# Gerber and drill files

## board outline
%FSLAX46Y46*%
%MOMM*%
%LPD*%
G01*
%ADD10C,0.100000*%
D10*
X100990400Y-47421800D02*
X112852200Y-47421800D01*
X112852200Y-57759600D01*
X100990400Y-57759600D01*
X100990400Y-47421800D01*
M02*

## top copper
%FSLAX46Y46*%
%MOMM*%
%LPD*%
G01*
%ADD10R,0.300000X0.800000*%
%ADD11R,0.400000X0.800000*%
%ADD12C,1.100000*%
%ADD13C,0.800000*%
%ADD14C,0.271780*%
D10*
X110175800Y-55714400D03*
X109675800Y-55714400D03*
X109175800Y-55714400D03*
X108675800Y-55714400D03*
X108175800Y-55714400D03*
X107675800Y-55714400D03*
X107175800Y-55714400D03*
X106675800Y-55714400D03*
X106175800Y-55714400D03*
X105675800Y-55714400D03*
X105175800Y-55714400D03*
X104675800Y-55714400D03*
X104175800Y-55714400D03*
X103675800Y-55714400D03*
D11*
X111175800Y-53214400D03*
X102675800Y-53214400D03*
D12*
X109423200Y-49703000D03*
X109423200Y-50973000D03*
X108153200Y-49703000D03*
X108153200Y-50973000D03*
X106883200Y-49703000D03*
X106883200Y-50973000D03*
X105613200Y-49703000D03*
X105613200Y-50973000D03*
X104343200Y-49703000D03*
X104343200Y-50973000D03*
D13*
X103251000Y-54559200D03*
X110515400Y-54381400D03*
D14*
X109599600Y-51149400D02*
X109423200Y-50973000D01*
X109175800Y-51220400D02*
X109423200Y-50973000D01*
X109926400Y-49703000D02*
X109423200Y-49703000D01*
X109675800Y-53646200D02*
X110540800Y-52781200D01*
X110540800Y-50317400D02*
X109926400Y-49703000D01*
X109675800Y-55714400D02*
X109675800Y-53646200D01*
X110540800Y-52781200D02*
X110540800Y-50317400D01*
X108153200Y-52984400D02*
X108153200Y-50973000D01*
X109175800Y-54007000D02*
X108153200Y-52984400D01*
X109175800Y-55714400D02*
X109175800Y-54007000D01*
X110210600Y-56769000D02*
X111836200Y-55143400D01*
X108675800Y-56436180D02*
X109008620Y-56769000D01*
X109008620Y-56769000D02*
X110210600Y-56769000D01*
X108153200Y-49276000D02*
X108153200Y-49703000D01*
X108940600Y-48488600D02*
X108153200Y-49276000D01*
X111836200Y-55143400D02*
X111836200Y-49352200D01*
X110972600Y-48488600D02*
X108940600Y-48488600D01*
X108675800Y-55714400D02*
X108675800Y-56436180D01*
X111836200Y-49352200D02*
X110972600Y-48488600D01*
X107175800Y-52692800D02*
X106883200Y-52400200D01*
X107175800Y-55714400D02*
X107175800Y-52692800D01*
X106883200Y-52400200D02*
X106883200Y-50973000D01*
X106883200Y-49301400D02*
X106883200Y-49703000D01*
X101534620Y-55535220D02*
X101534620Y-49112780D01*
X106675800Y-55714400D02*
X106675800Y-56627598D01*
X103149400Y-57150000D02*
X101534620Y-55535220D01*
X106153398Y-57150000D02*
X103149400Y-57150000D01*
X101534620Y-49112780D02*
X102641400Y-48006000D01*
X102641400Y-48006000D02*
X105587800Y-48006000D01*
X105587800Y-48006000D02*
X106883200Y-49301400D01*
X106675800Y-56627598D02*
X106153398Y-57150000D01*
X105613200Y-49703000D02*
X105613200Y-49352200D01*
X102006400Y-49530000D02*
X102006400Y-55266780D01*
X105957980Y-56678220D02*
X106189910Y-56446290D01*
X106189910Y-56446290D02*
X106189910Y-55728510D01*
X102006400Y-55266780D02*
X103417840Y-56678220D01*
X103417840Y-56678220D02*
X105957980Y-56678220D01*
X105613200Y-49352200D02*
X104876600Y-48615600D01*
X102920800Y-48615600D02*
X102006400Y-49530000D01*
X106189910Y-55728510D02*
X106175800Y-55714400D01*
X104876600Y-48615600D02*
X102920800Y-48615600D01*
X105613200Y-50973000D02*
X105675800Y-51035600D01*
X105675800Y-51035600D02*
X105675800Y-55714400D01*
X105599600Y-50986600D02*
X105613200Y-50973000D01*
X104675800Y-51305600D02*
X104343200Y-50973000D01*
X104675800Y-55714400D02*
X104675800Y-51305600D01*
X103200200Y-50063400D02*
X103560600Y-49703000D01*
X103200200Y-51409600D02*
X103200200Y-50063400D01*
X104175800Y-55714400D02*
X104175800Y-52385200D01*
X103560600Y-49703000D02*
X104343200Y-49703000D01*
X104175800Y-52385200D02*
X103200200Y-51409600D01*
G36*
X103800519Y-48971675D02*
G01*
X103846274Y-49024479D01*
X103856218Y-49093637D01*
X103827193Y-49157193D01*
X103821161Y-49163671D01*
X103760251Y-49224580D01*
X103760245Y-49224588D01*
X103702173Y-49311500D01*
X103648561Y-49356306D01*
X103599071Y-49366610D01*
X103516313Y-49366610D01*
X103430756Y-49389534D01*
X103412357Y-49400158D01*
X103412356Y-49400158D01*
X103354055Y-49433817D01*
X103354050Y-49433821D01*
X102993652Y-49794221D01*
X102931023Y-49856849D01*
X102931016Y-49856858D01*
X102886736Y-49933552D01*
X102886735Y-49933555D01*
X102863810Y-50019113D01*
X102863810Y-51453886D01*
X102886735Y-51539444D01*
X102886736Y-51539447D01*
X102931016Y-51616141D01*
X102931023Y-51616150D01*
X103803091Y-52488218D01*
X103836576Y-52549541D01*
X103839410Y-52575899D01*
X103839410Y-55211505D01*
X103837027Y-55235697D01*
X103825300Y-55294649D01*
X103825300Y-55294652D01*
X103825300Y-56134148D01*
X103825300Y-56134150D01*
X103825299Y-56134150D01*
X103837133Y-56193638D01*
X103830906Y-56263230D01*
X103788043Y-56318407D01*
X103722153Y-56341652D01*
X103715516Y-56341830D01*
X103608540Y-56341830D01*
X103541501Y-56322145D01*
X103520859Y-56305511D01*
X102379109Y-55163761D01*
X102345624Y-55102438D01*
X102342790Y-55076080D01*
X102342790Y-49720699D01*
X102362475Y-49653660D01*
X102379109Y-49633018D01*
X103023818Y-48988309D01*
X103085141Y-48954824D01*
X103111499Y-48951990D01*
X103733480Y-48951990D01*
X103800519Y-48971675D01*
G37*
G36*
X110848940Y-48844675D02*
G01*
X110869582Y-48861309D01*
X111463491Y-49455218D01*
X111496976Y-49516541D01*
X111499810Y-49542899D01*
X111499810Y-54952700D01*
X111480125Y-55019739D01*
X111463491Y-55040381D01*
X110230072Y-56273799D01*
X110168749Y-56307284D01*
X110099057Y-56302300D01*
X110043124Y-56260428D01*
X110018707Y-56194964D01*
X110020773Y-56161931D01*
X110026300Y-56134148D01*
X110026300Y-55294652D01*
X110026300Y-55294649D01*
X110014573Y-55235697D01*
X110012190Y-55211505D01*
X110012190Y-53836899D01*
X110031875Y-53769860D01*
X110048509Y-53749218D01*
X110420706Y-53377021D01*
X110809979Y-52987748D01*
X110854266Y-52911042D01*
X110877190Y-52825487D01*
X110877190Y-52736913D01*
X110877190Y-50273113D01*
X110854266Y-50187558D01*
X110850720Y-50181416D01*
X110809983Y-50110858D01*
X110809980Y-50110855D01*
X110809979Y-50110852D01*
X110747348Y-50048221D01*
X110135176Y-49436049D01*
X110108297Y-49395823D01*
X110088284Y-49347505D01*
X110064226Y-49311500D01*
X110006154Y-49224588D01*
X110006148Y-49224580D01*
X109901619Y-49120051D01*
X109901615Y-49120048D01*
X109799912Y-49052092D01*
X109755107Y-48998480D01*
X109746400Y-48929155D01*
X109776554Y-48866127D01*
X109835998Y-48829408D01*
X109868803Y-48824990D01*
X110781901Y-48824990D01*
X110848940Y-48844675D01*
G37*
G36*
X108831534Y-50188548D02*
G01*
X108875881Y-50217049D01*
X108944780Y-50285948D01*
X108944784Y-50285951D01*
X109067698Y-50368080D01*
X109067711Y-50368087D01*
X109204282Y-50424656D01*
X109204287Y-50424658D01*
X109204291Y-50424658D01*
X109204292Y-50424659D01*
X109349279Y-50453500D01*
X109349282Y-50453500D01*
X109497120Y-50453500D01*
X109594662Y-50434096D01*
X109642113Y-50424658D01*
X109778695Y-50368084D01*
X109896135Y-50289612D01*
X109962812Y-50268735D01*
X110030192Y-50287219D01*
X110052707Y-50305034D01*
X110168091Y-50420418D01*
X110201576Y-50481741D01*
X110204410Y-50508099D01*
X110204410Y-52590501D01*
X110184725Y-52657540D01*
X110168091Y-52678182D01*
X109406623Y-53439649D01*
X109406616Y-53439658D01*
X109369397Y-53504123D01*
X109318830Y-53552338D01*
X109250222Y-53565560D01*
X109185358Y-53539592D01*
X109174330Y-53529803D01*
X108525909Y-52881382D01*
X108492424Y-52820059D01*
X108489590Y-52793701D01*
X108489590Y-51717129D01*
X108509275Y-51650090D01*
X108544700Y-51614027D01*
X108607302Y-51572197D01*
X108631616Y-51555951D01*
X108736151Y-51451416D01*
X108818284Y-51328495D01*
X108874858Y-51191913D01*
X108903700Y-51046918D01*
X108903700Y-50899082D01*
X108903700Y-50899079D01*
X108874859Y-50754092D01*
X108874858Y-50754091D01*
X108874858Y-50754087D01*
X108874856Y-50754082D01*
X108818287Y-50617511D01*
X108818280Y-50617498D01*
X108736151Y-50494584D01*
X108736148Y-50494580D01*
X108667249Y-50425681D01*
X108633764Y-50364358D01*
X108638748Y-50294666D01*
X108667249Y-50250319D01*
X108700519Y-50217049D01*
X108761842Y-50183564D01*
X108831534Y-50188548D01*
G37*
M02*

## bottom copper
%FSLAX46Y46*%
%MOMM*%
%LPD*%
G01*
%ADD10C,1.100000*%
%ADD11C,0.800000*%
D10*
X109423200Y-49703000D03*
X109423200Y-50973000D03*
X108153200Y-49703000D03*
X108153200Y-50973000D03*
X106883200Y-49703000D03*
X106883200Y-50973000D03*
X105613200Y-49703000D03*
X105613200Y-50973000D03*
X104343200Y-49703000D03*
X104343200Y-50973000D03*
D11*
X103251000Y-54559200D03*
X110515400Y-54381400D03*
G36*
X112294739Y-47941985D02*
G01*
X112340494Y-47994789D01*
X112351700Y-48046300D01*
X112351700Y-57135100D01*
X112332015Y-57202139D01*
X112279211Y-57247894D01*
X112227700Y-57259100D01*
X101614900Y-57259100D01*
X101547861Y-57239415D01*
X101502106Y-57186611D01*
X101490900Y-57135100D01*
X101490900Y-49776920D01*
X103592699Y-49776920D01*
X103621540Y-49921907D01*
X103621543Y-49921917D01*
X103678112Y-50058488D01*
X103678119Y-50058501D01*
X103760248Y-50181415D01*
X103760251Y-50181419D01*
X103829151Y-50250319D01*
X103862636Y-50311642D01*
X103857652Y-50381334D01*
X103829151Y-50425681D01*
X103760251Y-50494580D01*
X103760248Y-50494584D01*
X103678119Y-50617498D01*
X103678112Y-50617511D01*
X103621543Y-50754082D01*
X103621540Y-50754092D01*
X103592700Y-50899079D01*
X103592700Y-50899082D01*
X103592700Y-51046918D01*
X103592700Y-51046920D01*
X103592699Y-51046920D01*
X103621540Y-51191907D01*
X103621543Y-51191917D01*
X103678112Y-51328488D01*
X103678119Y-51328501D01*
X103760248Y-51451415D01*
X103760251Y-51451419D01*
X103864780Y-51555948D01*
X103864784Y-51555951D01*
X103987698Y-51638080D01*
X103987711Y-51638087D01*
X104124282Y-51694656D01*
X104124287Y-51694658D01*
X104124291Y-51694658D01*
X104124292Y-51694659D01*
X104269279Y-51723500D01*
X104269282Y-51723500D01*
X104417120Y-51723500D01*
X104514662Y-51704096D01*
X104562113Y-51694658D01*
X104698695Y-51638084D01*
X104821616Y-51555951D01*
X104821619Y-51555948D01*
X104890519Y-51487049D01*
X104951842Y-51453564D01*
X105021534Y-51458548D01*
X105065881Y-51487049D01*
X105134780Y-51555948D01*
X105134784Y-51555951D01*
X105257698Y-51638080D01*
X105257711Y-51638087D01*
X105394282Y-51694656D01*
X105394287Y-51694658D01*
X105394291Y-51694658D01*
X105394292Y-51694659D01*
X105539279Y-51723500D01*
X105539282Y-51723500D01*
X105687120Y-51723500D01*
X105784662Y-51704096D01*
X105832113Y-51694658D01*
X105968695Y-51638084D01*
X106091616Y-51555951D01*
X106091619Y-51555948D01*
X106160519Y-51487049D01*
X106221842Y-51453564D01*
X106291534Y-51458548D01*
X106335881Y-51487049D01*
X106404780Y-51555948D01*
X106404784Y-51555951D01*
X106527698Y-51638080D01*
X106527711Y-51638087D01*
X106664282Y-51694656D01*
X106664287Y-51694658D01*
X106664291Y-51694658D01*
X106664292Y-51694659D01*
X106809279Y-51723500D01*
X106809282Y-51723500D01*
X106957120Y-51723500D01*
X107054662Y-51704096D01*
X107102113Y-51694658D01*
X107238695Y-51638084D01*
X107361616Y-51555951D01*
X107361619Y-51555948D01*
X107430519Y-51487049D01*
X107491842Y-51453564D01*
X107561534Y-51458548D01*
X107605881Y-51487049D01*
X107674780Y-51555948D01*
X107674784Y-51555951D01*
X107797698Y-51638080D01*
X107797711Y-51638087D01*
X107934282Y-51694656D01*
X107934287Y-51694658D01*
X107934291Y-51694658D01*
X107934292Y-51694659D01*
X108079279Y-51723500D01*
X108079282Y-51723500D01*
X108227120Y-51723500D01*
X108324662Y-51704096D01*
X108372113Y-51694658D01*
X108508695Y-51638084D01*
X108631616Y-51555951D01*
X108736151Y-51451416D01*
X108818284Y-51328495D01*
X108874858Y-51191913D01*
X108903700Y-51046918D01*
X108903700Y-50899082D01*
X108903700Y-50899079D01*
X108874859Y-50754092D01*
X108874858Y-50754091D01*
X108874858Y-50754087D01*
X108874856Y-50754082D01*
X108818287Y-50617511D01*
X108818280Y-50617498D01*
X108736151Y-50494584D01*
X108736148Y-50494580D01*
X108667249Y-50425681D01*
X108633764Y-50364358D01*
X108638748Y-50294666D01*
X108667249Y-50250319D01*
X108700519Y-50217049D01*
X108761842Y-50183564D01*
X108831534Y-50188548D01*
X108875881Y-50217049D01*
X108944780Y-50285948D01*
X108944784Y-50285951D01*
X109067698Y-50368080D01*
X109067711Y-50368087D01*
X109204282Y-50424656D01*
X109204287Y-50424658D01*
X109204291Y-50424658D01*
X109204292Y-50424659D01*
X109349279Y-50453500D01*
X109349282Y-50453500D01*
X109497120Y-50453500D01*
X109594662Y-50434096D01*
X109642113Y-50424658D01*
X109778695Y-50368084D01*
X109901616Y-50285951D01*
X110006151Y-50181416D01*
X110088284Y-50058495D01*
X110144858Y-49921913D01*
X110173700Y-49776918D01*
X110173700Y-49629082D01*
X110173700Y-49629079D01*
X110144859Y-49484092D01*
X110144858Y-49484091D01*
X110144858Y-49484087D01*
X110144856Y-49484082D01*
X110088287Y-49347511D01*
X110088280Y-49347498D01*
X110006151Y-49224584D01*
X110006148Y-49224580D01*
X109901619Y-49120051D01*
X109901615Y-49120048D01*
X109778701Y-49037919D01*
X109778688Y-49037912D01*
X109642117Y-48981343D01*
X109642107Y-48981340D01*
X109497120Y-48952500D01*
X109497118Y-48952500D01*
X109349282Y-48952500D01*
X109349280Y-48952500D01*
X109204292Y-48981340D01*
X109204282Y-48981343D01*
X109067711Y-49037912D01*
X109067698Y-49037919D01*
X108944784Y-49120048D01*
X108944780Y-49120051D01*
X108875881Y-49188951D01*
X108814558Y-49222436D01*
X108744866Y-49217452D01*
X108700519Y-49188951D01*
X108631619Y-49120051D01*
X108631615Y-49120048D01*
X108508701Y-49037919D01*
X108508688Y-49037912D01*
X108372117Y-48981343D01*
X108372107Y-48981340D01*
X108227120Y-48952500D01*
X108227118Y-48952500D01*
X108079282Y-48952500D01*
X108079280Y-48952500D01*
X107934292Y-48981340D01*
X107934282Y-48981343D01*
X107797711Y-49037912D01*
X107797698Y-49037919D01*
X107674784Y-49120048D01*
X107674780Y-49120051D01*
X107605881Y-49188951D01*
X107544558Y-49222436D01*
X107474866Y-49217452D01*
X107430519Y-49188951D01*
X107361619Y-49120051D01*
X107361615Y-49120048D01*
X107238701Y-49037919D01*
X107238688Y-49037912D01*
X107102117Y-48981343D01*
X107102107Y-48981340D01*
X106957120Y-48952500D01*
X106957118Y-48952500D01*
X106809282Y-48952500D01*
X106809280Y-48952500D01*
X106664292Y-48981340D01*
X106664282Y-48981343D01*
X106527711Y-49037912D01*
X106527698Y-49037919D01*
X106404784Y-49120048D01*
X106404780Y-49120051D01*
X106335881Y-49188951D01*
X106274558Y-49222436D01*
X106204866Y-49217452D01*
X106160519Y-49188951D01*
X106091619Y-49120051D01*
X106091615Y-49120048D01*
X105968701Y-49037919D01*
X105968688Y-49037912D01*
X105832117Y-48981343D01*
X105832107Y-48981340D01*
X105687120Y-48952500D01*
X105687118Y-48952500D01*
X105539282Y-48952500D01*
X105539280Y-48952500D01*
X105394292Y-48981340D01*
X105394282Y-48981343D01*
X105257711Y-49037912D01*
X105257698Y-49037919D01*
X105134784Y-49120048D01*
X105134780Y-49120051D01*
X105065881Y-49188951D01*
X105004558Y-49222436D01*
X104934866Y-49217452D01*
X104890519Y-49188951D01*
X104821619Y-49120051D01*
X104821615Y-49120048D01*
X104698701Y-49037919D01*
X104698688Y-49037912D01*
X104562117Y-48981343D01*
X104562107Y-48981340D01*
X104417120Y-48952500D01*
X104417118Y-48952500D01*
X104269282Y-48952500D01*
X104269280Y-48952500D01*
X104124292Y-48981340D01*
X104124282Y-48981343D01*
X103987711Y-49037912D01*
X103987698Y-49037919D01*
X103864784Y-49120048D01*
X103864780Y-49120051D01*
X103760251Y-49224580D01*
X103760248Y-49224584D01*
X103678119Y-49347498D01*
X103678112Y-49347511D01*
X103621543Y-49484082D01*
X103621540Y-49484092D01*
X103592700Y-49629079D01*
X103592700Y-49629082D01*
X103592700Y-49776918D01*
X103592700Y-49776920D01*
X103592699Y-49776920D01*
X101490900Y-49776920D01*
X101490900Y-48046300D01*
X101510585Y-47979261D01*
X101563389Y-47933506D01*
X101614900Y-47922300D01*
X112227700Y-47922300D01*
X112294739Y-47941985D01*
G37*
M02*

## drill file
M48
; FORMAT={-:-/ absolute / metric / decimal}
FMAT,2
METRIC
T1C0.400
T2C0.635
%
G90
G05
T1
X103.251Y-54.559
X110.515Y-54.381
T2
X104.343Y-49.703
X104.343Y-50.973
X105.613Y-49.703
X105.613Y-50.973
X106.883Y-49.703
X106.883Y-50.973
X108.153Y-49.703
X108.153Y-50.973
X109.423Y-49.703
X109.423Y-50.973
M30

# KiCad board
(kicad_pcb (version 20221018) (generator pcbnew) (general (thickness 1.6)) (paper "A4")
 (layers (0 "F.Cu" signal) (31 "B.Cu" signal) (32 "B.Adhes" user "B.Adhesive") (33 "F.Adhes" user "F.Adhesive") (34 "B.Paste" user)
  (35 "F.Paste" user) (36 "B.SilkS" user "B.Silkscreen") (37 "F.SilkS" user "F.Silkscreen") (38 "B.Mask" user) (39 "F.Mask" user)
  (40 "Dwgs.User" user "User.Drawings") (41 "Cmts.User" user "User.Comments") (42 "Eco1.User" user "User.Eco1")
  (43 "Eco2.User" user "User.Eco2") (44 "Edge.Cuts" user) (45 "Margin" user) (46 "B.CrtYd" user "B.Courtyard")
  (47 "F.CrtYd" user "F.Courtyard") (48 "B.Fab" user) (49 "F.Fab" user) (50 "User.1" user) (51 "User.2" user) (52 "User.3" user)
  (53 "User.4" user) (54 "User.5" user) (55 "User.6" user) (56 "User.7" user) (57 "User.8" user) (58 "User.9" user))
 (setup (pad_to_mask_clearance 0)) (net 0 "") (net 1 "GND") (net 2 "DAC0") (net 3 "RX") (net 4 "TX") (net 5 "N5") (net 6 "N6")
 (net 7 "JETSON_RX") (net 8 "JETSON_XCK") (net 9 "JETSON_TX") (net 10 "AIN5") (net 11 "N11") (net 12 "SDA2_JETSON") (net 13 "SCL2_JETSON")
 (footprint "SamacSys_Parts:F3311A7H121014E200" (layer "F.Cu") (at 106.9258 54.3694 180)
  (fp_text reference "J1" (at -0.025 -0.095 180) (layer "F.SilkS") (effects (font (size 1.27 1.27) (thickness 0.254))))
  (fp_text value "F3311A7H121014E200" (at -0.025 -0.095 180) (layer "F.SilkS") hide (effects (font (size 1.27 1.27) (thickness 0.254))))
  (pad "1" smd rect (at -3.25 -1.345 180) (size 0.3 0.8) (layers "F.Cu" "F.Paste" "F.Mask") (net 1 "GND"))
  (pad "2" smd rect (at -2.75 -1.345 180) (size 0.3 0.8) (layers "F.Cu" "F.Paste" "F.Mask") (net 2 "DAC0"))
  (pad "3" smd rect (at -2.25 -1.345 180) (size 0.3 0.8) (layers "F.Cu" "F.Paste" "F.Mask") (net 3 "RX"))
  (pad "4" smd rect (at -1.75 -1.345 180) (size 0.3 0.8) (layers "F.Cu" "F.Paste" "F.Mask") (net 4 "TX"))
  (pad "5" smd rect (at -1.25 -1.345 180) (size 0.3 0.8) (layers "F.Cu" "F.Paste" "F.Mask") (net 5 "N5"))
  (pad "6" smd rect (at -0.75 -1.345 180) (size 0.3 0.8) (layers "F.Cu" "F.Paste" "F.Mask") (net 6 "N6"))
  (pad "7" smd rect (at -0.25 -1.345 180) (size 0.3 0.8) (layers "F.Cu" "F.Paste" "F.Mask") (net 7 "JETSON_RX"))
  (pad "8" smd rect (at 0.25 -1.345 180) (size 0.3 0.8) (layers "F.Cu" "F.Paste" "F.Mask") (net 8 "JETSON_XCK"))
  (pad "9" smd rect (at 0.75 -1.345 180) (size 0.3 0.8) (layers "F.Cu" "F.Paste" "F.Mask") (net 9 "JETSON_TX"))
  (pad "10" smd rect (at 1.25 -1.345 180) (size 0.3 0.8) (layers "F.Cu" "F.Paste" "F.Mask") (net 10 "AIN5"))
  (pad "11" smd rect (at 1.75 -1.345 180) (size 0.3 0.8) (layers "F.Cu" "F.Paste" "F.Mask") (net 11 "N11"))
  (pad "12" smd rect (at 2.25 -1.345 180) (size 0.3 0.8) (layers "F.Cu" "F.Paste" "F.Mask") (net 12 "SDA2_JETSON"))
  (pad "13" smd rect (at 2.75 -1.345 180) (size 0.3 0.8) (layers "F.Cu" "F.Paste" "F.Mask") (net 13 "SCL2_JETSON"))
  (pad "14" smd rect (at 3.25 -1.345 180) (size 0.3 0.8) (layers "F.Cu" "F.Paste" "F.Mask") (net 1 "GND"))
  (pad "MP1" smd rect (at -4.25 1.155 180) (size 0.4 0.8) (layers "F.Cu" "F.Paste" "F.Mask") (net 1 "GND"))
  (pad "MP2" smd rect (at 4.25 1.155 180) (size 0.4 0.8) (layers "F.Cu" "F.Paste" "F.Mask") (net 1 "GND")))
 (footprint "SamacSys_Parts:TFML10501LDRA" (layer "F.Cu") (at 109.4232 49.703)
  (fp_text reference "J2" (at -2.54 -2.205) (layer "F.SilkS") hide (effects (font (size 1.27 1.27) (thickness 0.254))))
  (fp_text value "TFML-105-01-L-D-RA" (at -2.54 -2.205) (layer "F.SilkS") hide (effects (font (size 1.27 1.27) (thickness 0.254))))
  (pad "1" thru_hole circle (at 0 0) (size 1.1 1.1) (drill 0.635) (layers "*.Cu" "*.Mask") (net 2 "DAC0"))
  (pad "2" thru_hole circle (at 0 1.27) (size 1.1 1.1) (drill 0.635) (layers "*.Cu" "*.Mask") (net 1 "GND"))
  (pad "3" thru_hole circle (at -1.27 0) (size 1.1 1.1) (drill 0.635) (layers "*.Cu" "*.Mask") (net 4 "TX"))
  (pad "4" thru_hole circle (at -1.27 1.27) (size 1.1 1.1) (drill 0.635) (layers "*.Cu" "*.Mask") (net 3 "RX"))
  (pad "5" thru_hole circle (at -2.54 0) (size 1.1 1.1) (drill 0.635) (layers "*.Cu" "*.Mask") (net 8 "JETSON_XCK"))
  (pad "6" thru_hole circle (at -2.54 1.27) (size 1.1 1.1) (drill 0.635) (layers "*.Cu" "*.Mask") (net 7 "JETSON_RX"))
  (pad "7" thru_hole circle (at -3.81 0) (size 1.1 1.1) (drill 0.635) (layers "*.Cu" "*.Mask") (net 9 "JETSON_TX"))
  (pad "8" thru_hole circle (at -3.81 1.27) (size 1.1 1.1) (drill 0.635) (layers "*.Cu" "*.Mask") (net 10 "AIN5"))
  (pad "9" thru_hole circle (at -5.08 0) (size 1.1 1.1) (drill 0.635) (layers "*.Cu" "*.Mask") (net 13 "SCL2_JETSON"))
  (pad "10" thru_hole circle (at -5.08 1.27) (size 1.1 1.1) (drill 0.635) (layers "*.Cu" "*.Mask") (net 12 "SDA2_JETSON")))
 (gr_rect (start 100.9904 47.4218) (end 112.8522 57.7596) (stroke (width 0.1) (type default)) (fill none) (layer "Edge.Cuts"))
 (segment (start 109.5996 51.1494) (end 109.4232 50.973) (width 0.27178) (layer "F.Cu") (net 1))
 (segment (start 109.1758 51.2204) (end 109.4232 50.973) (width 0.27178) (layer "F.Cu") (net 1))
 (via (at 103.251 54.5592) (size 0.8) (drill 0.4) (layers "F.Cu" "B.Cu") (free) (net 1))
 (via (at 110.5154 54.3814) (size 0.8) (drill 0.4) (layers "F.Cu" "B.Cu") (free) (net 1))
 (segment (start 109.9264 49.703) (end 109.4232 49.703) (width 0.27178) (layer "F.Cu") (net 2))
 (segment (start 109.6758 53.6462) (end 110.5408 52.7812) (width 0.27178) (layer "F.Cu") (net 2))
 (segment (start 110.5408 50.3174) (end 109.9264 49.703) (width 0.27178) (layer "F.Cu") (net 2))
 (segment (start 109.6758 55.7144) (end 109.6758 53.6462) (width 0.27178) (layer "F.Cu") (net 2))
 (segment (start 110.5408 52.7812) (end 110.5408 50.3174) (width 0.27178) (layer "F.Cu") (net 2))
 (segment (start 108.1532 52.9844) (end 108.1532 50.973) (width 0.27178) (layer "F.Cu") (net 3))
 (segment (start 109.1758 54.007) (end 108.1532 52.9844) (width 0.27178) (layer "F.Cu") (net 3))
 (segment (start 109.1758 55.7144) (end 109.1758 54.007) (width 0.27178) (layer "F.Cu") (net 3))
 (segment (start 110.2106 56.769) (end 111.8362 55.1434) (width 0.27178) (layer "F.Cu") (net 4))
 (segment (start 108.6758 56.43618) (end 109.00862 56.769) (width 0.27178) (layer "F.Cu") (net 4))
 (segment (start 109.00862 56.769) (end 110.2106 56.769) (width 0.27178) (layer "F.Cu") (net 4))
 (segment (start 108.1532 49.276) (end 108.1532 49.703) (width 0.27178) (layer "F.Cu") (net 4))
 (segment (start 108.9406 48.4886) (end 108.1532 49.276) (width 0.27178) (layer "F.Cu") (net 4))
 (segment (start 111.8362 55.1434) (end 111.8362 49.3522) (width 0.27178) (layer "F.Cu") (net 4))
 (segment (start 110.9726 48.4886) (end 108.9406 48.4886) (width 0.27178) (layer "F.Cu") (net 4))
 (segment (start 108.6758 55.7144) (end 108.6758 56.43618) (width 0.27178) (layer "F.Cu") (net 4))
 (segment (start 111.8362 49.3522) (end 110.9726 48.4886) (width 0.27178) (layer "F.Cu") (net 4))
 (segment (start 107.1758 52.6928) (end 106.8832 52.4002) (width 0.27178) (layer "F.Cu") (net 7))
 (segment (start 107.1758 55.7144) (end 107.1758 52.6928) (width 0.27178) (layer "F.Cu") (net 7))
 (segment (start 106.8832 52.4002) (end 106.8832 50.973) (width 0.27178) (layer "F.Cu") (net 7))
 (segment (start 106.8832 49.3014) (end 106.8832 49.703) (width 0.27178) (layer "F.Cu") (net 8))
 (segment (start 101.53462 55.53522) (end 101.53462 49.11278) (width 0.27178) (layer "F.Cu") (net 8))
 (segment (start 106.6758 55.7144) (end 106.6758 56.627598) (width 0.27178) (layer "F.Cu") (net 8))
 (segment (start 103.1494 57.15) (end 101.53462 55.53522) (width 0.27178) (layer "F.Cu") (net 8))
 (segment (start 106.153398 57.15) (end 103.1494 57.15) (width 0.27178) (layer "F.Cu") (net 8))
 (segment (start 101.53462 49.11278) (end 102.6414 48.006) (width 0.27178) (layer "F.Cu") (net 8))
 (segment (start 102.6414 48.006) (end 105.5878 48.006) (width 0.27178) (layer "F.Cu") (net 8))
 (segment (start 105.5878 48.006) (end 106.8832 49.3014) (width 0.27178) (layer "F.Cu") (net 8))
 (segment (start 106.6758 56.627598) (end 106.153398 57.15) (width 0.27178) (layer "F.Cu") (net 8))
 (segment (start 105.6132 49.703) (end 105.6132 49.3522) (width 0.27178) (layer "F.Cu") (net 9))
 (segment (start 102.0064 49.53) (end 102.0064 55.26678) (width 0.27178) (layer "F.Cu") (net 9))
 (segment (start 105.95798 56.67822) (end 106.18991 56.44629) (width 0.27178) (layer "F.Cu") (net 9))
 (segment (start 106.18991 56.44629) (end 106.18991 55.72851) (width 0.27178) (layer "F.Cu") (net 9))
 (segment (start 102.0064 55.26678) (end 103.41784 56.67822) (width 0.27178) (layer "F.Cu") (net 9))
 (segment (start 103.41784 56.67822) (end 105.95798 56.67822) (width 0.27178) (layer "F.Cu") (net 9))
 (segment (start 105.6132 49.3522) (end 104.8766 48.6156) (width 0.27178) (layer "F.Cu") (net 9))
 (segment (start 102.9208 48.6156) (end 102.0064 49.53) (width 0.27178) (layer "F.Cu") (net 9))
 (segment (start 106.18991 55.72851) (end 106.1758 55.7144) (width 0.27178) (layer "F.Cu") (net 9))
 (segment (start 104.8766 48.6156) (end 102.9208 48.6156) (width 0.27178) (layer "F.Cu") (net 9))
 (segment (start 105.6132 50.973) (end 105.6758 51.0356) (width 0.27178) (layer "F.Cu") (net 10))
 (segment (start 105.6758 51.0356) (end 105.6758 55.7144) (width 0.27178) (layer "F.Cu") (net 10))
 (segment (start 105.5996 50.9866) (end 105.6132 50.973) (width 0.27178) (layer "F.Cu") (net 10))
 (segment (start 104.6758 51.3056) (end 104.3432 50.973) (width 0.27178) (layer "F.Cu") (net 12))
 (segment (start 104.6758 55.7144) (end 104.6758 51.3056) (width 0.27178) (layer "F.Cu") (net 12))
 (segment (start 103.2002 50.0634) (end 103.5606 49.703) (width 0.27178) (layer "F.Cu") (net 13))
 (segment (start 103.2002 51.4096) (end 103.2002 50.0634) (width 0.27178) (layer "F.Cu") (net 13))
 (segment (start 104.1758 55.7144) (end 104.1758 52.3852) (width 0.27178) (layer "F.Cu") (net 13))
 (segment (start 103.5606 49.703) (end 104.3432 49.703) (width 0.27178) (layer "F.Cu") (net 13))
 (segment (start 104.1758 52.3852) (end 103.2002 51.4096) (width 0.27178) (layer "F.Cu") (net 13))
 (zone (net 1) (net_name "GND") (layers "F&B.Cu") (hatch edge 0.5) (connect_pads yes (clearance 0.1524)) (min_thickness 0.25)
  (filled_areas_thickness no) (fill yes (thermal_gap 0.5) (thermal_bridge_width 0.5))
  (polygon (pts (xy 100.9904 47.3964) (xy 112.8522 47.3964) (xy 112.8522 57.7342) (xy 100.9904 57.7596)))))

